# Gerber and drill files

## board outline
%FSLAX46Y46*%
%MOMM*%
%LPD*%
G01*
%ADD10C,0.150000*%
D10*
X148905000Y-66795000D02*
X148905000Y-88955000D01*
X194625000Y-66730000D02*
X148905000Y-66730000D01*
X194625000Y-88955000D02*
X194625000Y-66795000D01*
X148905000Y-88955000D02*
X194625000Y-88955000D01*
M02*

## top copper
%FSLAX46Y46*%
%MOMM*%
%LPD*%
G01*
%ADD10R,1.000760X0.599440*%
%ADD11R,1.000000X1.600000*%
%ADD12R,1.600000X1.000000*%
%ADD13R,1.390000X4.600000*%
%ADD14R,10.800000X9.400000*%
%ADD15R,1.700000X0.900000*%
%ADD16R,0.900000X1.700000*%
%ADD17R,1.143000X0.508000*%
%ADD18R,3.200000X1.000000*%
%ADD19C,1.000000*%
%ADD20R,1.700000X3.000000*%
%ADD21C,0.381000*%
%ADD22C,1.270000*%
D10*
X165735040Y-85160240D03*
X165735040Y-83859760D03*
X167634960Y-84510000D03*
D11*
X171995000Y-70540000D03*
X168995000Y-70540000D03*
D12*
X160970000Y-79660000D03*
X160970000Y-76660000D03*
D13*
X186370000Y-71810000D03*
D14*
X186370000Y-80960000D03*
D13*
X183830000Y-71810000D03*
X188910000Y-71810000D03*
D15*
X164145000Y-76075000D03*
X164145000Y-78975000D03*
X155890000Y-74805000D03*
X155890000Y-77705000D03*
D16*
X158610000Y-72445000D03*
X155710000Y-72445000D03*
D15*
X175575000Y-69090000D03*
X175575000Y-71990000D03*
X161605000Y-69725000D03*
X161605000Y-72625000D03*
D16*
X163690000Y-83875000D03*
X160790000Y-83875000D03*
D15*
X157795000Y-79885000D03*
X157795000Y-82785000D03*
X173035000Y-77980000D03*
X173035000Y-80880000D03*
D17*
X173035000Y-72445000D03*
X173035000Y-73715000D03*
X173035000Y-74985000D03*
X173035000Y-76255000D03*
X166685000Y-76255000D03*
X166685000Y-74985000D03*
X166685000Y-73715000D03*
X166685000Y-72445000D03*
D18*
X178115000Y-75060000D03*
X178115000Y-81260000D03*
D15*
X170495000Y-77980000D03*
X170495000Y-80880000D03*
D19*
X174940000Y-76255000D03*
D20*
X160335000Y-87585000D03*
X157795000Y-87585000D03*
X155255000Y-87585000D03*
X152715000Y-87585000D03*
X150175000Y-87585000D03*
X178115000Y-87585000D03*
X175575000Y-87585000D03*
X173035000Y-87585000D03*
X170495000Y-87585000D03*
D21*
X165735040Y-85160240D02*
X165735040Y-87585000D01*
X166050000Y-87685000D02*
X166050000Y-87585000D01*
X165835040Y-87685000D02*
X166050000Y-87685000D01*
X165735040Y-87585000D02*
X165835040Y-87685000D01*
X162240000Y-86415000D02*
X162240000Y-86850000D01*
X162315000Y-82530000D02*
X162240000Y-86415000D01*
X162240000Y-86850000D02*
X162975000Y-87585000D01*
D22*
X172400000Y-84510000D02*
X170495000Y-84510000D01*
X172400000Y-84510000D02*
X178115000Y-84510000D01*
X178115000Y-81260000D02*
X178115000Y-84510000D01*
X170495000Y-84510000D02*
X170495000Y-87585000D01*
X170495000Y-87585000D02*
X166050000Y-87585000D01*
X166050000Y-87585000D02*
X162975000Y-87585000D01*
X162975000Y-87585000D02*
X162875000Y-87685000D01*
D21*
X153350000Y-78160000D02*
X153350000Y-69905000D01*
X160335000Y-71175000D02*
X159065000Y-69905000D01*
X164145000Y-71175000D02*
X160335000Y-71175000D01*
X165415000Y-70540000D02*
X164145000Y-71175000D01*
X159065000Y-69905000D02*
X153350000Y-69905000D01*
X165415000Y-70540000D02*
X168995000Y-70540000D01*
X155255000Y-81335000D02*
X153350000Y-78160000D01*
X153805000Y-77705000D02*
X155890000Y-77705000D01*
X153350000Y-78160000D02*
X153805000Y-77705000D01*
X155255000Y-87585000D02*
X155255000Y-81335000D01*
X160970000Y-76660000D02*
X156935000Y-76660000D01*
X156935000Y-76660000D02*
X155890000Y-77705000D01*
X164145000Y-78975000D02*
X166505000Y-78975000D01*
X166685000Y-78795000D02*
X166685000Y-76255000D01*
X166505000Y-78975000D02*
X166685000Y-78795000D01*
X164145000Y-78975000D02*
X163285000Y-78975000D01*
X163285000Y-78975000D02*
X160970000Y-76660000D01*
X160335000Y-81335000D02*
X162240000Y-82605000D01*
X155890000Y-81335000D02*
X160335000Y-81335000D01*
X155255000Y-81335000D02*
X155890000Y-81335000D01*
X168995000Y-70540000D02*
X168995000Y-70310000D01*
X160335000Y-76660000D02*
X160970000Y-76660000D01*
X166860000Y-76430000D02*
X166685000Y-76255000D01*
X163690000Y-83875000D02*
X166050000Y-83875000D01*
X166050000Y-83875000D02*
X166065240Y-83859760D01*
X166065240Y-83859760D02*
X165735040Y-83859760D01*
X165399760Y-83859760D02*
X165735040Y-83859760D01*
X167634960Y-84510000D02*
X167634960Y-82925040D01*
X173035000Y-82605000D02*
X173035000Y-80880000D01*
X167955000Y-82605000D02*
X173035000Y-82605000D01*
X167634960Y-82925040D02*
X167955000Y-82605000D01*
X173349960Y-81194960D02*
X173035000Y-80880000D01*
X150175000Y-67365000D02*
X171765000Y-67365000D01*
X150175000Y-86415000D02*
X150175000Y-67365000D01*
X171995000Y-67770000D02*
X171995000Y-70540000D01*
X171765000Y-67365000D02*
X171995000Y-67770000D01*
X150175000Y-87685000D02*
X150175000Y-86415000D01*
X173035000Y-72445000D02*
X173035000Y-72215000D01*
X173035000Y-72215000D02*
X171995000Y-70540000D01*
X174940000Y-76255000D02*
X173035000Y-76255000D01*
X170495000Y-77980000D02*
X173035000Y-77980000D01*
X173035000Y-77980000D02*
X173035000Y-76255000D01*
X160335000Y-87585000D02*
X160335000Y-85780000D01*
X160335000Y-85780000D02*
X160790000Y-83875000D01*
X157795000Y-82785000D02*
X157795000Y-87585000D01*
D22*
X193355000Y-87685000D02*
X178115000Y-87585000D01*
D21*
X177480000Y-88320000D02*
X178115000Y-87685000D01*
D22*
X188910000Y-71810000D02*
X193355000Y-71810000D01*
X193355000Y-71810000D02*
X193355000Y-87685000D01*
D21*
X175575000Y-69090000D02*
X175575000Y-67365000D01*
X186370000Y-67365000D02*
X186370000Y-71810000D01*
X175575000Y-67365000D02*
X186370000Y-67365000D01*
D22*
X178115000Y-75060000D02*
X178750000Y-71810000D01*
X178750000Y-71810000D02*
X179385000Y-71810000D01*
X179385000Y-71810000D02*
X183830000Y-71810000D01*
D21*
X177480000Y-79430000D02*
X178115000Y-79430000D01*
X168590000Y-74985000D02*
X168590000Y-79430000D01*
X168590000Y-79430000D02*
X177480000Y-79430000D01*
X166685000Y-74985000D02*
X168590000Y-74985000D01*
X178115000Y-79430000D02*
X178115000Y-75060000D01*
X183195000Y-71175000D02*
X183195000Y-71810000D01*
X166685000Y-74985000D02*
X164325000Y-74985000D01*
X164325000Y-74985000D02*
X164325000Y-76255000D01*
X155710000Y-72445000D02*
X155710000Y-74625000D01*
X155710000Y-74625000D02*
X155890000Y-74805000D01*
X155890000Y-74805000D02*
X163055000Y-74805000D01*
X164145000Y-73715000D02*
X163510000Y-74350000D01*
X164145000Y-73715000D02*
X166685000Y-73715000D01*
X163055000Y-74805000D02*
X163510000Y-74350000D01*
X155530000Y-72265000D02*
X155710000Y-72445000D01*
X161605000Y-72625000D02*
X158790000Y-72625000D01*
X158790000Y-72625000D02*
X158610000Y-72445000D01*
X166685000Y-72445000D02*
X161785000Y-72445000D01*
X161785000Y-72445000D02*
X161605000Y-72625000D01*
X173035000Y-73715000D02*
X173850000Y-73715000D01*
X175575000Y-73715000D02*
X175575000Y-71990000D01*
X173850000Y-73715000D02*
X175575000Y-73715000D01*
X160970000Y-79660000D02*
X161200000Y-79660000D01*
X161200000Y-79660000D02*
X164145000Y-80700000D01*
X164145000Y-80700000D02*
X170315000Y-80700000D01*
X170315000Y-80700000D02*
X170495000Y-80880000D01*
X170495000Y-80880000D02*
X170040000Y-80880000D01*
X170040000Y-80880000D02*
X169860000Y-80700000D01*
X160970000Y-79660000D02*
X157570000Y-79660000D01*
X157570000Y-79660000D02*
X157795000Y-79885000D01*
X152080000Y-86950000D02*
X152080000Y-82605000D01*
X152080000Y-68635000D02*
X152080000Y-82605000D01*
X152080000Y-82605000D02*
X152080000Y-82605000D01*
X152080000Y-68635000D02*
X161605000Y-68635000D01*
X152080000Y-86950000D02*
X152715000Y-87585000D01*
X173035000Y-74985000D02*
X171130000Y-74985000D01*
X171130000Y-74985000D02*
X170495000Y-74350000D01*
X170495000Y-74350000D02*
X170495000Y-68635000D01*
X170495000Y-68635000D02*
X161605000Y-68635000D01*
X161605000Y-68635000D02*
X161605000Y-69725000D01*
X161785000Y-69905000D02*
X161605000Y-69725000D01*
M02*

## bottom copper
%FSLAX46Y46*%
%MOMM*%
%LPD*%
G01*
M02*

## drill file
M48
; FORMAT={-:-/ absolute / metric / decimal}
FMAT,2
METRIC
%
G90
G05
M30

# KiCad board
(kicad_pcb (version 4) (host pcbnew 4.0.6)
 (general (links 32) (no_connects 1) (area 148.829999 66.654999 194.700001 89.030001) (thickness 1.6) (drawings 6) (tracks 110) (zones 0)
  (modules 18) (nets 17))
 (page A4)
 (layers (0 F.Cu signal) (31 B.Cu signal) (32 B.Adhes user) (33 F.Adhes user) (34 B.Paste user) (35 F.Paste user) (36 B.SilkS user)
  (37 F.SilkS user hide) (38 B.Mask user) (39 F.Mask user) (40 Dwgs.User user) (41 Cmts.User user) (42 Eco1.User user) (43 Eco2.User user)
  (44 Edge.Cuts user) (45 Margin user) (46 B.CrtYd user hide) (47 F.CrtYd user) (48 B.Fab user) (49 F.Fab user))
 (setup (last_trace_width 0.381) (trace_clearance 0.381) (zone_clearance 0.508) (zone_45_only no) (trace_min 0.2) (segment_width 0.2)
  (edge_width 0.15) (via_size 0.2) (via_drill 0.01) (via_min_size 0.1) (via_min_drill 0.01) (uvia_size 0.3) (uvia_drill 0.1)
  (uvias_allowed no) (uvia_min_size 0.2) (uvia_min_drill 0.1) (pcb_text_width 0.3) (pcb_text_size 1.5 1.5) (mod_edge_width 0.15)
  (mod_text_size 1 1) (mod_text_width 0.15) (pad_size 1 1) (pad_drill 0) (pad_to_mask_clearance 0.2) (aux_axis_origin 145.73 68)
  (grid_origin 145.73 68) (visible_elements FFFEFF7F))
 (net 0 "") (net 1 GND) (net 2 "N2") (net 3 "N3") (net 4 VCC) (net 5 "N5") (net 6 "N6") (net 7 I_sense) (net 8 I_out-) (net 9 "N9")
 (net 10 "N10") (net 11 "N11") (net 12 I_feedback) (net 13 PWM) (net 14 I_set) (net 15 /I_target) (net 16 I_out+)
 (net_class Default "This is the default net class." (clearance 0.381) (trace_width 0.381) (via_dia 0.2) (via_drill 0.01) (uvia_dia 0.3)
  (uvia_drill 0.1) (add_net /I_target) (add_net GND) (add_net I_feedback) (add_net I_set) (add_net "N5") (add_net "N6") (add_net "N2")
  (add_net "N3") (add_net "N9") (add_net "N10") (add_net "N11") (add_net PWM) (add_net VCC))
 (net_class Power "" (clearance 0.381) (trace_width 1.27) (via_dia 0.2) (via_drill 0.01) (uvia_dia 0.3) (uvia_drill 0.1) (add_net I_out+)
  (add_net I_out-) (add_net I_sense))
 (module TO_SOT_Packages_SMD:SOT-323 (layer F.Cu) (at 166.685 84.51 90)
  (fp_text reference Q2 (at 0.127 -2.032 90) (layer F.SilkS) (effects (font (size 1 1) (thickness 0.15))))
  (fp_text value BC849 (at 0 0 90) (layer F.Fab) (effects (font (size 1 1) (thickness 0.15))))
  (pad 2 smd rect (at -0.65024 -0.94996 90) (size 0.59944 1.00076) (layers F.Cu F.Paste F.Mask) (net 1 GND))
  (pad 1 smd rect (at 0.65024 -0.94996 90) (size 0.59944 1.00076) (layers F.Cu F.Paste F.Mask) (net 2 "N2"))
  (pad 3 smd rect (at 0 0.94996 90) (size 0.59944 1.00076) (layers F.Cu F.Paste F.Mask) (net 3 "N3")))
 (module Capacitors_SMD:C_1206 (layer F.Cu) (at 170.495 70.54 180)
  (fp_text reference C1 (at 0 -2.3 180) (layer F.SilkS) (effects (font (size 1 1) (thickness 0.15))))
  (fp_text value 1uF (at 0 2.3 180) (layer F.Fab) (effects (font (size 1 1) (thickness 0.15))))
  (pad 1 smd rect (at -1.5 0 180) (size 1 1.6) (layers F.Cu F.Paste F.Mask) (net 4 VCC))
  (pad 2 smd rect (at 1.5 0 180) (size 1 1.6) (layers F.Cu F.Paste F.Mask) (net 1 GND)))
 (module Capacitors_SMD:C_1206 (layer F.Cu) (at 160.97 78.16 90)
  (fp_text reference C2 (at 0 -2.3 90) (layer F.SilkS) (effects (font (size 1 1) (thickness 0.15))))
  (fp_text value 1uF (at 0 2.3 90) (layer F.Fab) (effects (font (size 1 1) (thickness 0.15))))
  (pad 1 smd rect (at -1.5 0 90) (size 1 1.6) (layers F.Cu F.Paste F.Mask) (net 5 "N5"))
  (pad 2 smd rect (at 1.5 0 90) (size 1 1.6) (layers F.Cu F.Paste F.Mask) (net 1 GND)))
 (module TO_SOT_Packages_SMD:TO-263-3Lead (layer F.Cu) (at 186.37 71.81 270)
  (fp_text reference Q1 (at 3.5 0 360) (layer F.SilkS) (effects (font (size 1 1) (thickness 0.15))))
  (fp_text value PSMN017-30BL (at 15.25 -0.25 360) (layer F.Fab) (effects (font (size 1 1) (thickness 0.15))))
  (pad 2 smd rect (at 0 0 270) (size 4.6 1.39) (layers F.Cu F.Paste F.Mask) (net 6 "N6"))
  (pad 4 smd rect (at 9.15 0 270) (size 9.4 10.8) (layers F.Cu F.Paste F.Mask))
  (pad 3 smd rect (at 0 2.54 270) (size 4.6 1.39) (layers F.Cu F.Paste F.Mask) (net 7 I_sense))
  (pad 1 smd rect (at 0 -2.54 270) (size 4.6 1.39) (layers F.Cu F.Paste F.Mask) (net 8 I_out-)))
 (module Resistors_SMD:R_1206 (layer F.Cu) (at 164.145 77.525 270)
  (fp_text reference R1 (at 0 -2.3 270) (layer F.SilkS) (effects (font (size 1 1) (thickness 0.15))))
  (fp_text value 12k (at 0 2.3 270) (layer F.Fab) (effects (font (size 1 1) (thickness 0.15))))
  (pad 1 smd rect (at -1.45 0 270) (size 0.9 1.7) (layers F.Cu F.Paste F.Mask) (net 7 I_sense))
  (pad 2 smd rect (at 1.45 0 270) (size 0.9 1.7) (layers F.Cu F.Paste F.Mask) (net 1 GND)))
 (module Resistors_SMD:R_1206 (layer F.Cu) (at 155.89 76.255 270)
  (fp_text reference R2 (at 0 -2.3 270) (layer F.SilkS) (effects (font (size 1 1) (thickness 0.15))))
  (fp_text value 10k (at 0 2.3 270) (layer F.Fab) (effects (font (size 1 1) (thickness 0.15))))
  (pad 1 smd rect (at -1.45 0 270) (size 0.9 1.7) (layers F.Cu F.Paste F.Mask) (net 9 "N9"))
  (pad 2 smd rect (at 1.45 0 270) (size 0.9 1.7) (layers F.Cu F.Paste F.Mask) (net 1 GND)))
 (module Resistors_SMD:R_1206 (layer F.Cu) (at 157.16 72.445 180)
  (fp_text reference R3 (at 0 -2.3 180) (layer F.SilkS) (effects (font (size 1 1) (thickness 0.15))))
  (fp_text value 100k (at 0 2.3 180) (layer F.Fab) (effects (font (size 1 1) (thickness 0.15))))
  (pad 1 smd rect (at -1.45 0 180) (size 0.9 1.7) (layers F.Cu F.Paste F.Mask) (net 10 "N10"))
  (pad 2 smd rect (at 1.45 0 180) (size 0.9 1.7) (layers F.Cu F.Paste F.Mask) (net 9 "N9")))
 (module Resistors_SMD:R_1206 (layer F.Cu) (at 175.575 70.54 270)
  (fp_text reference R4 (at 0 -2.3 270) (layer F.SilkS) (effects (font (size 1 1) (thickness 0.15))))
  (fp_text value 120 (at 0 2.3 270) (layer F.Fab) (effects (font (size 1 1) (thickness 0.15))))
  (pad 1 smd rect (at -1.45 0 270) (size 0.9 1.7) (layers F.Cu F.Paste F.Mask) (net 6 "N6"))
  (pad 2 smd rect (at 1.45 0 270) (size 0.9 1.7) (layers F.Cu F.Paste F.Mask) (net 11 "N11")))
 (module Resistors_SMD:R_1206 (layer F.Cu) (at 161.605 71.175 270)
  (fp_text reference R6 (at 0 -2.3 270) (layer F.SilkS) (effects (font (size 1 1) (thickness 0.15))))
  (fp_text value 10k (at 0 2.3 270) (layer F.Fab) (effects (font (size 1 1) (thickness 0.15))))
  (pad 1 smd rect (at -1.45 0 270) (size 0.9 1.7) (layers F.Cu F.Paste F.Mask) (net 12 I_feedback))
  (pad 2 smd rect (at 1.45 0 270) (size 0.9 1.7) (layers F.Cu F.Paste F.Mask) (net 10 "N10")))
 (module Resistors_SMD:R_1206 (layer F.Cu) (at 162.24 83.875 180)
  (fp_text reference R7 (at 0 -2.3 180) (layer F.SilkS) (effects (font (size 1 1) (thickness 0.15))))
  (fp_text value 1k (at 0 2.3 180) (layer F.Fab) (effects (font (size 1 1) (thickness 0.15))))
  (pad 1 smd rect (at -1.45 0 180) (size 0.9 1.7) (layers F.Cu F.Paste F.Mask) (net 2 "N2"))
  (pad 2 smd rect (at 1.45 0 180) (size 0.9 1.7) (layers F.Cu F.Paste F.Mask) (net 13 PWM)))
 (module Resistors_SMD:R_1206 (layer F.Cu) (at 157.795 81.335 270)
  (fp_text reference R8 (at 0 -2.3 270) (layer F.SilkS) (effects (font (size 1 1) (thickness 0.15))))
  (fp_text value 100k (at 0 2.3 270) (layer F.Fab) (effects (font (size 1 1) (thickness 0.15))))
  (pad 1 smd rect (at -1.45 0 270) (size 0.9 1.7) (layers F.Cu F.Paste F.Mask) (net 5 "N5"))
  (pad 2 smd rect (at 1.45 0 270) (size 0.9 1.7) (layers F.Cu F.Paste F.Mask) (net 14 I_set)))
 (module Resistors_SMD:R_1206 (layer F.Cu) (at 173.035 79.43 270)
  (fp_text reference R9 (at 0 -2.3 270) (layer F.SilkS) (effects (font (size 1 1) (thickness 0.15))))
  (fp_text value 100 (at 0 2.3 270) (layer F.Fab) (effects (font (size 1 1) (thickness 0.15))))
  (pad 1 smd rect (at -1.45 0 270) (size 0.9 1.7) (layers F.Cu F.Paste F.Mask) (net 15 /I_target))
  (pad 2 smd rect (at 1.45 0 270) (size 0.9 1.7) (layers F.Cu F.Paste F.Mask) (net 3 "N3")))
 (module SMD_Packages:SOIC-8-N (layer F.Cu) (at 169.86 74.35 270)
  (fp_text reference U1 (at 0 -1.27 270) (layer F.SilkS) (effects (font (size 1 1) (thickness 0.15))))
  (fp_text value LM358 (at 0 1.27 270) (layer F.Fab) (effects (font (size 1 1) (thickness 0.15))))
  (pad 8 smd rect (at -1.905 -3.175 270) (size 0.508 1.143) (layers F.Cu F.Paste F.Mask) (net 4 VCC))
  (pad 7 smd rect (at -0.635 -3.175 270) (size 0.508 1.143) (layers F.Cu F.Paste F.Mask) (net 11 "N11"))
  (pad 6 smd rect (at 0.635 -3.175 270) (size 0.508 1.143) (layers F.Cu F.Paste F.Mask) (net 12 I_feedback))
  (pad 5 smd rect (at 1.905 -3.175 270) (size 0.508 1.143) (layers F.Cu F.Paste F.Mask) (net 15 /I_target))
  (pad 4 smd rect (at 1.905 3.175 270) (size 0.508 1.143) (layers F.Cu F.Paste F.Mask) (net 1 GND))
  (pad 3 smd rect (at 0.635 3.175 270) (size 0.508 1.143) (layers F.Cu F.Paste F.Mask) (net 7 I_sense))
  (pad 2 smd rect (at -0.635 3.175 270) (size 0.508 1.143) (layers F.Cu F.Paste F.Mask) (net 9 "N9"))
  (pad 1 smd rect (at -1.905 3.175 270) (size 0.508 1.143) (layers F.Cu F.Paste F.Mask) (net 10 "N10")))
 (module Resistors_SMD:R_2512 (layer F.Cu) (at 178.115 78.16 270)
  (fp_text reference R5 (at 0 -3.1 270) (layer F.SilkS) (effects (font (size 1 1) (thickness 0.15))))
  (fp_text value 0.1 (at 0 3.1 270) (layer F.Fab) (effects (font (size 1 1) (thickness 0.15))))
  (pad 1 smd rect (at -3.1 0 270) (size 1 3.2) (layers F.Cu F.Paste F.Mask) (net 7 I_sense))
  (pad 2 smd rect (at 3.1 0 270) (size 1 3.2) (layers F.Cu F.Paste F.Mask) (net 1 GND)))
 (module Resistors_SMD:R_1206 (layer F.Cu) (at 170.495 79.43 270)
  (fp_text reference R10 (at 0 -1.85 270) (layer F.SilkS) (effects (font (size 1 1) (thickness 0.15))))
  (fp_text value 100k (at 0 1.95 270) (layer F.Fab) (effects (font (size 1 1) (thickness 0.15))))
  (pad 1 smd rect (at -1.45 0 270) (size 0.9 1.7) (layers F.Cu F.Paste F.Mask) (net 15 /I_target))
  (pad 2 smd rect (at 1.45 0 270) (size 0.9 1.7) (layers F.Cu F.Paste F.Mask) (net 5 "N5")))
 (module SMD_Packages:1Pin (layer F.Cu) (at 174.94 76.255)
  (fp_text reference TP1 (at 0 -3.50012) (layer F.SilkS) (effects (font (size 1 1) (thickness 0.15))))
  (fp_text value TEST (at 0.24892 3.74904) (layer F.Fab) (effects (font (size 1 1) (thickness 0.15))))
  (pad 1 smd circle (at 0 0) (size 1 1) (layers F.Cu F.Paste F.Mask) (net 15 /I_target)))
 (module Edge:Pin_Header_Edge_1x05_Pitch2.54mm (layer F.Cu) (at 160.335 87.685 270)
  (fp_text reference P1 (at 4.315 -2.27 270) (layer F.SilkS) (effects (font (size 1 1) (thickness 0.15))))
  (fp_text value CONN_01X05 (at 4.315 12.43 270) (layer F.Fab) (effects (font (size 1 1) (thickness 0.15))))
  (pad 1 smd rect (at -0.1 0 270) (size 3 1.7) (layers F.Cu F.Paste F.Mask) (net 13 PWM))
  (pad 2 smd rect (at -0.1 2.54 270) (size 3 1.7) (layers F.Cu F.Paste F.Mask) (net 14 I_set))
  (pad 3 smd rect (at -0.1 5.08 270) (size 3 1.7) (layers F.Cu F.Paste F.Mask) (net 1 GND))
  (pad 4 smd rect (at -0.1 7.62 270) (size 3 1.7) (layers F.Cu F.Paste F.Mask) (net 12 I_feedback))
  (pad 5 smd rect (at -0.1 10.16 270) (size 3 1.7) (layers F.Cu F.Paste F.Mask) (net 4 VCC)))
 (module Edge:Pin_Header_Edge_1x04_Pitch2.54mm (layer F.Cu) (at 178.115 87.685 270)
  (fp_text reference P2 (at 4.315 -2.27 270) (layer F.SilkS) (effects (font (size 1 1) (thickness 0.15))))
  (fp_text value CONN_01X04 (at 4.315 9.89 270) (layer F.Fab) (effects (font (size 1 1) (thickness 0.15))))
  (pad 1 smd rect (at -0.1 0 270) (size 3 1.7) (layers F.Cu F.Paste F.Mask) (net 8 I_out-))
  (pad 2 smd rect (at -0.1 2.54 270) (size 3 1.7) (layers F.Cu F.Paste F.Mask) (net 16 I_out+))
  (pad 3 smd rect (at -0.1 5.08 270) (size 3 1.7) (layers F.Cu F.Paste F.Mask) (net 16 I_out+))
  (pad 4 smd rect (at -0.1 7.62 270) (size 3 1.7) (layers F.Cu F.Paste F.Mask) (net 1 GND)))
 (gr_line (start 148.905 66.795) (end 148.905 88.955) (angle 90) (layer Edge.Cuts) (width 0.15))
 (gr_line (start 194.625 66.73) (end 148.905 66.73) (angle 90) (layer Edge.Cuts) (width 0.15))
 (gr_line (start 194.625 88.955) (end 194.625 66.795) (angle 90) (layer Edge.Cuts) (width 0.15))
 (gr_line (start 148.905 88.955) (end 194.625 88.955) (angle 90) (layer Edge.Cuts) (width 0.15))
 (segment (start 165.73504 85.16024) (end 165.73504 87.585) (width 0.381) (layer F.Cu) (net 1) (status 400000))
 (segment (start 166.05 87.685) (end 166.05 87.585) (width 0.381) (layer F.Cu) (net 1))
 (segment (start 165.83504 87.685) (end 166.05 87.685) (width 0.381) (layer F.Cu) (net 1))
 (segment (start 165.73504 87.585) (end 165.83504 87.685) (width 0.381) (layer F.Cu) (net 1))
 (segment (start 162.24 86.415) (end 162.24 86.85) (width 0.381) (layer F.Cu) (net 1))
 (segment (start 162.315 82.53) (end 162.24 86.415) (width 0.381) (layer F.Cu) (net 1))
 (segment (start 162.24 86.85) (end 162.975 87.585) (width 0.381) (layer F.Cu) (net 1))
 (segment (start 172.4 84.51) (end 170.495 84.51) (width 1.27) (layer F.Cu) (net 1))
 (segment (start 172.4 84.51) (end 178.115 84.51) (width 1.27) (layer F.Cu) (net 1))
 (segment (start 178.115 81.26) (end 178.115 84.51) (width 1.27) (layer F.Cu) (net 1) (status 20))
 (segment (start 170.495 84.51) (end 170.495 87.585) (width 1.27) (layer F.Cu) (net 1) (status 800000))
 (segment (start 170.495 87.585) (end 166.05 87.585) (width 1.27) (layer F.Cu) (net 1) (status 400000))
 (segment (start 166.05 87.585) (end 162.975 87.585) (width 1.27) (layer F.Cu) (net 1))
 (segment (start 162.975 87.585) (end 162.875 87.685) (width 1.27) (layer F.Cu) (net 1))
 (segment (start 153.35 78.16) (end 153.35 69.905) (width 0.381) (layer F.Cu) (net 1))
 (segment (start 160.335 71.175) (end 159.065 69.905) (width 0.381) (layer F.Cu) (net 1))
 (segment (start 164.145 71.175) (end 160.335 71.175) (width 0.381) (layer F.Cu) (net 1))
 (segment (start 165.415 70.54) (end 164.145 71.175) (width 0.381) (layer F.Cu) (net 1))
 (segment (start 159.065 69.905) (end 153.35 69.905) (width 0.381) (layer F.Cu) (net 1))
 (segment (start 165.415 70.54) (end 168.995 70.54) (width 0.381) (layer F.Cu) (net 1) (status 20))
 (segment (start 155.255 81.335) (end 153.35 78.16) (width 0.381) (layer F.Cu) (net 1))
 (segment (start 153.805 77.705) (end 155.89 77.705) (width 0.381) (layer F.Cu) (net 1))
 (segment (start 153.35 78.16) (end 153.805 77.705) (width 0.381) (layer F.Cu) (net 1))
 (segment (start 155.255 87.585) (end 155.255 81.335) (width 0.381) (layer F.Cu) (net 1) (status 10))
 (segment (start 160.97 76.66) (end 156.935 76.66) (width 0.381) (layer F.Cu) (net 1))
 (segment (start 156.935 76.66) (end 155.89 77.705) (width 0.381) (layer F.Cu) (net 1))
 (segment (start 164.145 78.975) (end 166.505 78.975) (width 0.381) (layer F.Cu) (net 1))
 (segment (start 166.685 78.795) (end 166.685 76.255) (width 0.381) (layer F.Cu) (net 1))
 (segment (start 166.505 78.975) (end 166.685 78.795) (width 0.381) (layer F.Cu) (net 1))
 (segment (start 164.145 78.975) (end 163.285 78.975) (width 0.381) (layer F.Cu) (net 1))
 (segment (start 163.285 78.975) (end 160.97 76.66) (width 0.381) (layer F.Cu) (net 1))
 (segment (start 160.335 81.335) (end 162.24 82.605) (width 0.381) (layer F.Cu) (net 1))
 (segment (start 155.89 81.335) (end 160.335 81.335) (width 0.381) (layer F.Cu) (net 1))
 (segment (start 155.255 81.335) (end 155.89 81.335) (width 0.381) (layer F.Cu) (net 1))
 (segment (start 168.995 70.54) (end 168.995 70.31) (width 0.381) (layer F.Cu) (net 1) (status 30))
 (segment (start 160.335 76.66) (end 160.97 76.66) (width 0.381) (layer F.Cu) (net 1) (status 30))
 (segment (start 166.86 76.43) (end 166.685 76.255) (width 0.381) (layer F.Cu) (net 1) (status 30))
 (segment (start 163.69 83.875) (end 166.05 83.875) (width 0.381) (layer F.Cu) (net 2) (status 20))
 (segment (start 166.05 83.875) (end 166.06524 83.85976) (width 0.381) (layer F.Cu) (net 2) (status 30))
 (segment (start 166.06524 83.85976) (end 165.73504 83.85976) (width 0.381) (layer F.Cu) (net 2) (status 30))
 (segment (start 165.39976 83.85976) (end 165.73504 83.85976) (width 0.381) (layer F.Cu) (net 2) (status 30))
 (segment (start 167.63496 84.51) (end 167.63496 82.92504) (width 0.381) (layer F.Cu) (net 3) (status 400000))
 (segment (start 173.035 82.605) (end 173.035 80.88) (width 0.381) (layer F.Cu) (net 3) (status 800000))
 (segment (start 167.955 82.605) (end 173.035 82.605) (width 0.381) (layer F.Cu) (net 3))
 (segment (start 167.63496 82.92504) (end 167.955 82.605) (width 0.381) (layer F.Cu) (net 3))
 (segment (start 173.34996 81.19496) (end 173.035 80.88) (width 0.381) (layer F.Cu) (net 3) (status 30))
 (segment (start 150.175 67.365) (end 171.765 67.365) (width 0.381) (layer F.Cu) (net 4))
 (segment (start 150.175 86.415) (end 150.175 67.365) (width 0.381) (layer F.Cu) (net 4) (status 20))
 (segment (start 171.995 67.77) (end 171.995 70.54) (width 0.381) (layer F.Cu) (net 4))
 (segment (start 171.765 67.365) (end 171.995 67.77) (width 0.381) (layer F.Cu) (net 4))
 (segment (start 150.175 87.685) (end 150.175 86.415) (width 0.381) (layer F.Cu) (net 4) (status 30))
 (segment (start 173.035 72.445) (end 173.035 72.215) (width 0.381) (layer F.Cu) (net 4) (status 10))
 (segment (start 173.035 72.215) (end 171.995 70.54) (width 0.381) (layer F.Cu) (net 4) (status 20))
 (segment (start 174.94 76.255) (end 173.035 76.255) (width 0.381) (layer F.Cu) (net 15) (status 10))
 (segment (start 170.495 77.98) (end 173.035 77.98) (width 0.381) (layer F.Cu) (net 15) (status 10))
 (segment (start 173.035 77.98) (end 173.035 76.255) (width 0.381) (layer F.Cu) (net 15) (status 10))
 (segment (start 160.335 87.585) (end 160.335 85.78) (width 0.381) (layer F.Cu) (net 13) (status 10))
 (segment (start 160.335 85.78) (end 160.79 83.875) (width 0.381) (layer F.Cu) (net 13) (status 20))
 (segment (start 157.795 82.785) (end 157.795 87.585) (width 0.381) (layer F.Cu) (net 14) (status 10))
 (segment (start 193.355 87.685) (end 178.115 87.585) (width 1.27) (layer F.Cu) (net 8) (status 800000))
 (segment (start 177.48 88.32) (end 178.115 87.685) (width 0.381) (layer F.Cu) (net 8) (status 30))
 (segment (start 188.91 71.81) (end 193.355 71.81) (width 1.27) (layer F.Cu) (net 8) (status 10))
 (segment (start 193.355 71.81) (end 193.355 87.685) (width 1.27) (layer F.Cu) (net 8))
 (segment (start 175.575 69.09) (end 175.575 67.365) (width 0.381) (layer F.Cu) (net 6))
 (segment (start 186.37 67.365) (end 186.37 71.81) (width 0.381) (layer F.Cu) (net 6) (status 20))
 (segment (start 175.575 67.365) (end 186.37 67.365) (width 0.381) (layer F.Cu) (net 6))
 (segment (start 178.115 75.06) (end 178.75 71.81) (width 1.27) (layer F.Cu) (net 7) (status 10))
 (segment (start 178.75 71.81) (end 179.385 71.81) (width 1.27) (layer F.Cu) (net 7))
 (segment (start 179.385 71.81) (end 183.83 71.81) (width 1.27) (layer F.Cu) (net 7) (status 20))
 (segment (start 177.48 79.43) (end 178.115 79.43) (width 0.381) (layer F.Cu) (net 7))
 (segment (start 168.59 74.985) (end 168.59 79.43) (width 0.381) (layer F.Cu) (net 7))
 (segment (start 168.59 79.43) (end 177.48 79.43) (width 0.381) (layer F.Cu) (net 7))
 (segment (start 166.685 74.985) (end 168.59 74.985) (width 0.381) (layer F.Cu) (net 7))
 (segment (start 178.115 79.43) (end 178.115 75.06) (width 0.381) (layer F.Cu) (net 7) (status 20))
 (segment (start 183.195 71.175) (end 183.195 71.81) (width 0.381) (layer F.Cu) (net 7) (status 30))
 (segment (start 166.685 74.985) (end 164.325 74.985) (width 0.381) (layer F.Cu) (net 7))
 (segment (start 164.325 74.985) (end 164.325 76.255) (width 0.381) (layer F.Cu) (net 7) (status 20))
 (segment (start 155.71 72.445) (end 155.71 74.625) (width 0.381) (layer F.Cu) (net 9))
 (segment (start 155.71 74.625) (end 155.89 74.805) (width 0.381) (layer F.Cu) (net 9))
 (segment (start 155.89 74.805) (end 163.055 74.805) (width 0.381) (layer F.Cu) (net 9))
 (segment (start 164.145 73.715) (end 163.51 74.35) (width 0.381) (layer F.Cu) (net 9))
 (segment (start 164.145 73.715) (end 166.685 73.715) (width 0.381) (layer F.Cu) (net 9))
 (segment (start 163.055 74.805) (end 163.51 74.35) (width 0.381) (layer F.Cu) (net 9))
 (segment (start 155.53 72.265) (end 155.71 72.445) (width 0.381) (layer F.Cu) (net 9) (status 30))
 (segment (start 161.605 72.625) (end 158.79 72.625) (width 0.381) (layer F.Cu) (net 10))
 (segment (start 158.79 72.625) (end 158.61 72.445) (width 0.381) (layer F.Cu) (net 10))
 (segment (start 166.685 72.445) (end 161.785 72.445) (width 0.381) (layer F.Cu) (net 10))
 (segment (start 161.785 72.445) (end 161.605 72.625) (width 0.381) (layer F.Cu) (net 10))
 (segment (start 173.035 73.715) (end 173.85 73.715) (width 0.381) (layer F.Cu) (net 11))
 (segment (start 175.575 73.715) (end 175.575 71.99) (width 0.381) (layer F.Cu) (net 11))
 (segment (start 173.85 73.715) (end 175.575 73.715) (width 0.381) (layer F.Cu) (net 11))
 (segment (start 160.97 79.66) (end 161.2 79.66) (width 0.381) (layer F.Cu) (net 5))
 (segment (start 161.2 79.66) (end 164.145 80.7) (width 0.381) (layer F.Cu) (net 5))
 (segment (start 164.145 80.7) (end 170.315 80.7) (width 0.381) (layer F.Cu) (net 5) (status 20))
 (segment (start 170.315 80.7) (end 170.495 80.88) (width 0.381) (layer F.Cu) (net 5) (status 30))
 (segment (start 170.495 80.88) (end 170.04 80.88) (width 0.381) (layer F.Cu) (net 5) (status 30))
 (segment (start 170.04 80.88) (end 169.86 80.7) (width 0.381) (layer F.Cu) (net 5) (status 30))
 (segment (start 160.97 79.66) (end 157.57 79.66) (width 0.381) (layer F.Cu) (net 5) (status 20))
 (segment (start 157.57 79.66) (end 157.795 79.885) (width 0.381) (layer F.Cu) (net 5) (status 30))
 (segment (start 152.08 86.95) (end 152.08 82.605) (width 0.381) (layer F.Cu) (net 12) (status 10))
 (segment (start 152.08 68.635) (end 152.08 82.605) (width 0.381) (layer F.Cu) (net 12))
 (segment (start 152.08 82.605) (end 152.08 82.605) (width 0.381) (layer F.Cu) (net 12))
 (segment (start 152.08 68.635) (end 161.605 68.635) (width 0.381) (layer F.Cu) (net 12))
 (segment (start 152.08 86.95) (end 152.715 87.585) (width 0.381) (layer F.Cu) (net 12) (status 30))
 (segment (start 173.035 74.985) (end 171.13 74.985) (width 0.381) (layer F.Cu) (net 12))
 (segment (start 171.13 74.985) (end 170.495 74.35) (width 0.381) (layer F.Cu) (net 12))
 (segment (start 170.495 74.35) (end 170.495 68.635) (width 0.381) (layer F.Cu) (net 12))
 (segment (start 170.495 68.635) (end 161.605 68.635) (width 0.381) (layer F.Cu) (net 12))
 (segment (start 161.605 68.635) (end 161.605 69.725) (width 0.381) (layer F.Cu) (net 12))
 (segment (start 161.785 69.905) (end 161.605 69.725) (width 0.381) (layer F.Cu) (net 12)))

